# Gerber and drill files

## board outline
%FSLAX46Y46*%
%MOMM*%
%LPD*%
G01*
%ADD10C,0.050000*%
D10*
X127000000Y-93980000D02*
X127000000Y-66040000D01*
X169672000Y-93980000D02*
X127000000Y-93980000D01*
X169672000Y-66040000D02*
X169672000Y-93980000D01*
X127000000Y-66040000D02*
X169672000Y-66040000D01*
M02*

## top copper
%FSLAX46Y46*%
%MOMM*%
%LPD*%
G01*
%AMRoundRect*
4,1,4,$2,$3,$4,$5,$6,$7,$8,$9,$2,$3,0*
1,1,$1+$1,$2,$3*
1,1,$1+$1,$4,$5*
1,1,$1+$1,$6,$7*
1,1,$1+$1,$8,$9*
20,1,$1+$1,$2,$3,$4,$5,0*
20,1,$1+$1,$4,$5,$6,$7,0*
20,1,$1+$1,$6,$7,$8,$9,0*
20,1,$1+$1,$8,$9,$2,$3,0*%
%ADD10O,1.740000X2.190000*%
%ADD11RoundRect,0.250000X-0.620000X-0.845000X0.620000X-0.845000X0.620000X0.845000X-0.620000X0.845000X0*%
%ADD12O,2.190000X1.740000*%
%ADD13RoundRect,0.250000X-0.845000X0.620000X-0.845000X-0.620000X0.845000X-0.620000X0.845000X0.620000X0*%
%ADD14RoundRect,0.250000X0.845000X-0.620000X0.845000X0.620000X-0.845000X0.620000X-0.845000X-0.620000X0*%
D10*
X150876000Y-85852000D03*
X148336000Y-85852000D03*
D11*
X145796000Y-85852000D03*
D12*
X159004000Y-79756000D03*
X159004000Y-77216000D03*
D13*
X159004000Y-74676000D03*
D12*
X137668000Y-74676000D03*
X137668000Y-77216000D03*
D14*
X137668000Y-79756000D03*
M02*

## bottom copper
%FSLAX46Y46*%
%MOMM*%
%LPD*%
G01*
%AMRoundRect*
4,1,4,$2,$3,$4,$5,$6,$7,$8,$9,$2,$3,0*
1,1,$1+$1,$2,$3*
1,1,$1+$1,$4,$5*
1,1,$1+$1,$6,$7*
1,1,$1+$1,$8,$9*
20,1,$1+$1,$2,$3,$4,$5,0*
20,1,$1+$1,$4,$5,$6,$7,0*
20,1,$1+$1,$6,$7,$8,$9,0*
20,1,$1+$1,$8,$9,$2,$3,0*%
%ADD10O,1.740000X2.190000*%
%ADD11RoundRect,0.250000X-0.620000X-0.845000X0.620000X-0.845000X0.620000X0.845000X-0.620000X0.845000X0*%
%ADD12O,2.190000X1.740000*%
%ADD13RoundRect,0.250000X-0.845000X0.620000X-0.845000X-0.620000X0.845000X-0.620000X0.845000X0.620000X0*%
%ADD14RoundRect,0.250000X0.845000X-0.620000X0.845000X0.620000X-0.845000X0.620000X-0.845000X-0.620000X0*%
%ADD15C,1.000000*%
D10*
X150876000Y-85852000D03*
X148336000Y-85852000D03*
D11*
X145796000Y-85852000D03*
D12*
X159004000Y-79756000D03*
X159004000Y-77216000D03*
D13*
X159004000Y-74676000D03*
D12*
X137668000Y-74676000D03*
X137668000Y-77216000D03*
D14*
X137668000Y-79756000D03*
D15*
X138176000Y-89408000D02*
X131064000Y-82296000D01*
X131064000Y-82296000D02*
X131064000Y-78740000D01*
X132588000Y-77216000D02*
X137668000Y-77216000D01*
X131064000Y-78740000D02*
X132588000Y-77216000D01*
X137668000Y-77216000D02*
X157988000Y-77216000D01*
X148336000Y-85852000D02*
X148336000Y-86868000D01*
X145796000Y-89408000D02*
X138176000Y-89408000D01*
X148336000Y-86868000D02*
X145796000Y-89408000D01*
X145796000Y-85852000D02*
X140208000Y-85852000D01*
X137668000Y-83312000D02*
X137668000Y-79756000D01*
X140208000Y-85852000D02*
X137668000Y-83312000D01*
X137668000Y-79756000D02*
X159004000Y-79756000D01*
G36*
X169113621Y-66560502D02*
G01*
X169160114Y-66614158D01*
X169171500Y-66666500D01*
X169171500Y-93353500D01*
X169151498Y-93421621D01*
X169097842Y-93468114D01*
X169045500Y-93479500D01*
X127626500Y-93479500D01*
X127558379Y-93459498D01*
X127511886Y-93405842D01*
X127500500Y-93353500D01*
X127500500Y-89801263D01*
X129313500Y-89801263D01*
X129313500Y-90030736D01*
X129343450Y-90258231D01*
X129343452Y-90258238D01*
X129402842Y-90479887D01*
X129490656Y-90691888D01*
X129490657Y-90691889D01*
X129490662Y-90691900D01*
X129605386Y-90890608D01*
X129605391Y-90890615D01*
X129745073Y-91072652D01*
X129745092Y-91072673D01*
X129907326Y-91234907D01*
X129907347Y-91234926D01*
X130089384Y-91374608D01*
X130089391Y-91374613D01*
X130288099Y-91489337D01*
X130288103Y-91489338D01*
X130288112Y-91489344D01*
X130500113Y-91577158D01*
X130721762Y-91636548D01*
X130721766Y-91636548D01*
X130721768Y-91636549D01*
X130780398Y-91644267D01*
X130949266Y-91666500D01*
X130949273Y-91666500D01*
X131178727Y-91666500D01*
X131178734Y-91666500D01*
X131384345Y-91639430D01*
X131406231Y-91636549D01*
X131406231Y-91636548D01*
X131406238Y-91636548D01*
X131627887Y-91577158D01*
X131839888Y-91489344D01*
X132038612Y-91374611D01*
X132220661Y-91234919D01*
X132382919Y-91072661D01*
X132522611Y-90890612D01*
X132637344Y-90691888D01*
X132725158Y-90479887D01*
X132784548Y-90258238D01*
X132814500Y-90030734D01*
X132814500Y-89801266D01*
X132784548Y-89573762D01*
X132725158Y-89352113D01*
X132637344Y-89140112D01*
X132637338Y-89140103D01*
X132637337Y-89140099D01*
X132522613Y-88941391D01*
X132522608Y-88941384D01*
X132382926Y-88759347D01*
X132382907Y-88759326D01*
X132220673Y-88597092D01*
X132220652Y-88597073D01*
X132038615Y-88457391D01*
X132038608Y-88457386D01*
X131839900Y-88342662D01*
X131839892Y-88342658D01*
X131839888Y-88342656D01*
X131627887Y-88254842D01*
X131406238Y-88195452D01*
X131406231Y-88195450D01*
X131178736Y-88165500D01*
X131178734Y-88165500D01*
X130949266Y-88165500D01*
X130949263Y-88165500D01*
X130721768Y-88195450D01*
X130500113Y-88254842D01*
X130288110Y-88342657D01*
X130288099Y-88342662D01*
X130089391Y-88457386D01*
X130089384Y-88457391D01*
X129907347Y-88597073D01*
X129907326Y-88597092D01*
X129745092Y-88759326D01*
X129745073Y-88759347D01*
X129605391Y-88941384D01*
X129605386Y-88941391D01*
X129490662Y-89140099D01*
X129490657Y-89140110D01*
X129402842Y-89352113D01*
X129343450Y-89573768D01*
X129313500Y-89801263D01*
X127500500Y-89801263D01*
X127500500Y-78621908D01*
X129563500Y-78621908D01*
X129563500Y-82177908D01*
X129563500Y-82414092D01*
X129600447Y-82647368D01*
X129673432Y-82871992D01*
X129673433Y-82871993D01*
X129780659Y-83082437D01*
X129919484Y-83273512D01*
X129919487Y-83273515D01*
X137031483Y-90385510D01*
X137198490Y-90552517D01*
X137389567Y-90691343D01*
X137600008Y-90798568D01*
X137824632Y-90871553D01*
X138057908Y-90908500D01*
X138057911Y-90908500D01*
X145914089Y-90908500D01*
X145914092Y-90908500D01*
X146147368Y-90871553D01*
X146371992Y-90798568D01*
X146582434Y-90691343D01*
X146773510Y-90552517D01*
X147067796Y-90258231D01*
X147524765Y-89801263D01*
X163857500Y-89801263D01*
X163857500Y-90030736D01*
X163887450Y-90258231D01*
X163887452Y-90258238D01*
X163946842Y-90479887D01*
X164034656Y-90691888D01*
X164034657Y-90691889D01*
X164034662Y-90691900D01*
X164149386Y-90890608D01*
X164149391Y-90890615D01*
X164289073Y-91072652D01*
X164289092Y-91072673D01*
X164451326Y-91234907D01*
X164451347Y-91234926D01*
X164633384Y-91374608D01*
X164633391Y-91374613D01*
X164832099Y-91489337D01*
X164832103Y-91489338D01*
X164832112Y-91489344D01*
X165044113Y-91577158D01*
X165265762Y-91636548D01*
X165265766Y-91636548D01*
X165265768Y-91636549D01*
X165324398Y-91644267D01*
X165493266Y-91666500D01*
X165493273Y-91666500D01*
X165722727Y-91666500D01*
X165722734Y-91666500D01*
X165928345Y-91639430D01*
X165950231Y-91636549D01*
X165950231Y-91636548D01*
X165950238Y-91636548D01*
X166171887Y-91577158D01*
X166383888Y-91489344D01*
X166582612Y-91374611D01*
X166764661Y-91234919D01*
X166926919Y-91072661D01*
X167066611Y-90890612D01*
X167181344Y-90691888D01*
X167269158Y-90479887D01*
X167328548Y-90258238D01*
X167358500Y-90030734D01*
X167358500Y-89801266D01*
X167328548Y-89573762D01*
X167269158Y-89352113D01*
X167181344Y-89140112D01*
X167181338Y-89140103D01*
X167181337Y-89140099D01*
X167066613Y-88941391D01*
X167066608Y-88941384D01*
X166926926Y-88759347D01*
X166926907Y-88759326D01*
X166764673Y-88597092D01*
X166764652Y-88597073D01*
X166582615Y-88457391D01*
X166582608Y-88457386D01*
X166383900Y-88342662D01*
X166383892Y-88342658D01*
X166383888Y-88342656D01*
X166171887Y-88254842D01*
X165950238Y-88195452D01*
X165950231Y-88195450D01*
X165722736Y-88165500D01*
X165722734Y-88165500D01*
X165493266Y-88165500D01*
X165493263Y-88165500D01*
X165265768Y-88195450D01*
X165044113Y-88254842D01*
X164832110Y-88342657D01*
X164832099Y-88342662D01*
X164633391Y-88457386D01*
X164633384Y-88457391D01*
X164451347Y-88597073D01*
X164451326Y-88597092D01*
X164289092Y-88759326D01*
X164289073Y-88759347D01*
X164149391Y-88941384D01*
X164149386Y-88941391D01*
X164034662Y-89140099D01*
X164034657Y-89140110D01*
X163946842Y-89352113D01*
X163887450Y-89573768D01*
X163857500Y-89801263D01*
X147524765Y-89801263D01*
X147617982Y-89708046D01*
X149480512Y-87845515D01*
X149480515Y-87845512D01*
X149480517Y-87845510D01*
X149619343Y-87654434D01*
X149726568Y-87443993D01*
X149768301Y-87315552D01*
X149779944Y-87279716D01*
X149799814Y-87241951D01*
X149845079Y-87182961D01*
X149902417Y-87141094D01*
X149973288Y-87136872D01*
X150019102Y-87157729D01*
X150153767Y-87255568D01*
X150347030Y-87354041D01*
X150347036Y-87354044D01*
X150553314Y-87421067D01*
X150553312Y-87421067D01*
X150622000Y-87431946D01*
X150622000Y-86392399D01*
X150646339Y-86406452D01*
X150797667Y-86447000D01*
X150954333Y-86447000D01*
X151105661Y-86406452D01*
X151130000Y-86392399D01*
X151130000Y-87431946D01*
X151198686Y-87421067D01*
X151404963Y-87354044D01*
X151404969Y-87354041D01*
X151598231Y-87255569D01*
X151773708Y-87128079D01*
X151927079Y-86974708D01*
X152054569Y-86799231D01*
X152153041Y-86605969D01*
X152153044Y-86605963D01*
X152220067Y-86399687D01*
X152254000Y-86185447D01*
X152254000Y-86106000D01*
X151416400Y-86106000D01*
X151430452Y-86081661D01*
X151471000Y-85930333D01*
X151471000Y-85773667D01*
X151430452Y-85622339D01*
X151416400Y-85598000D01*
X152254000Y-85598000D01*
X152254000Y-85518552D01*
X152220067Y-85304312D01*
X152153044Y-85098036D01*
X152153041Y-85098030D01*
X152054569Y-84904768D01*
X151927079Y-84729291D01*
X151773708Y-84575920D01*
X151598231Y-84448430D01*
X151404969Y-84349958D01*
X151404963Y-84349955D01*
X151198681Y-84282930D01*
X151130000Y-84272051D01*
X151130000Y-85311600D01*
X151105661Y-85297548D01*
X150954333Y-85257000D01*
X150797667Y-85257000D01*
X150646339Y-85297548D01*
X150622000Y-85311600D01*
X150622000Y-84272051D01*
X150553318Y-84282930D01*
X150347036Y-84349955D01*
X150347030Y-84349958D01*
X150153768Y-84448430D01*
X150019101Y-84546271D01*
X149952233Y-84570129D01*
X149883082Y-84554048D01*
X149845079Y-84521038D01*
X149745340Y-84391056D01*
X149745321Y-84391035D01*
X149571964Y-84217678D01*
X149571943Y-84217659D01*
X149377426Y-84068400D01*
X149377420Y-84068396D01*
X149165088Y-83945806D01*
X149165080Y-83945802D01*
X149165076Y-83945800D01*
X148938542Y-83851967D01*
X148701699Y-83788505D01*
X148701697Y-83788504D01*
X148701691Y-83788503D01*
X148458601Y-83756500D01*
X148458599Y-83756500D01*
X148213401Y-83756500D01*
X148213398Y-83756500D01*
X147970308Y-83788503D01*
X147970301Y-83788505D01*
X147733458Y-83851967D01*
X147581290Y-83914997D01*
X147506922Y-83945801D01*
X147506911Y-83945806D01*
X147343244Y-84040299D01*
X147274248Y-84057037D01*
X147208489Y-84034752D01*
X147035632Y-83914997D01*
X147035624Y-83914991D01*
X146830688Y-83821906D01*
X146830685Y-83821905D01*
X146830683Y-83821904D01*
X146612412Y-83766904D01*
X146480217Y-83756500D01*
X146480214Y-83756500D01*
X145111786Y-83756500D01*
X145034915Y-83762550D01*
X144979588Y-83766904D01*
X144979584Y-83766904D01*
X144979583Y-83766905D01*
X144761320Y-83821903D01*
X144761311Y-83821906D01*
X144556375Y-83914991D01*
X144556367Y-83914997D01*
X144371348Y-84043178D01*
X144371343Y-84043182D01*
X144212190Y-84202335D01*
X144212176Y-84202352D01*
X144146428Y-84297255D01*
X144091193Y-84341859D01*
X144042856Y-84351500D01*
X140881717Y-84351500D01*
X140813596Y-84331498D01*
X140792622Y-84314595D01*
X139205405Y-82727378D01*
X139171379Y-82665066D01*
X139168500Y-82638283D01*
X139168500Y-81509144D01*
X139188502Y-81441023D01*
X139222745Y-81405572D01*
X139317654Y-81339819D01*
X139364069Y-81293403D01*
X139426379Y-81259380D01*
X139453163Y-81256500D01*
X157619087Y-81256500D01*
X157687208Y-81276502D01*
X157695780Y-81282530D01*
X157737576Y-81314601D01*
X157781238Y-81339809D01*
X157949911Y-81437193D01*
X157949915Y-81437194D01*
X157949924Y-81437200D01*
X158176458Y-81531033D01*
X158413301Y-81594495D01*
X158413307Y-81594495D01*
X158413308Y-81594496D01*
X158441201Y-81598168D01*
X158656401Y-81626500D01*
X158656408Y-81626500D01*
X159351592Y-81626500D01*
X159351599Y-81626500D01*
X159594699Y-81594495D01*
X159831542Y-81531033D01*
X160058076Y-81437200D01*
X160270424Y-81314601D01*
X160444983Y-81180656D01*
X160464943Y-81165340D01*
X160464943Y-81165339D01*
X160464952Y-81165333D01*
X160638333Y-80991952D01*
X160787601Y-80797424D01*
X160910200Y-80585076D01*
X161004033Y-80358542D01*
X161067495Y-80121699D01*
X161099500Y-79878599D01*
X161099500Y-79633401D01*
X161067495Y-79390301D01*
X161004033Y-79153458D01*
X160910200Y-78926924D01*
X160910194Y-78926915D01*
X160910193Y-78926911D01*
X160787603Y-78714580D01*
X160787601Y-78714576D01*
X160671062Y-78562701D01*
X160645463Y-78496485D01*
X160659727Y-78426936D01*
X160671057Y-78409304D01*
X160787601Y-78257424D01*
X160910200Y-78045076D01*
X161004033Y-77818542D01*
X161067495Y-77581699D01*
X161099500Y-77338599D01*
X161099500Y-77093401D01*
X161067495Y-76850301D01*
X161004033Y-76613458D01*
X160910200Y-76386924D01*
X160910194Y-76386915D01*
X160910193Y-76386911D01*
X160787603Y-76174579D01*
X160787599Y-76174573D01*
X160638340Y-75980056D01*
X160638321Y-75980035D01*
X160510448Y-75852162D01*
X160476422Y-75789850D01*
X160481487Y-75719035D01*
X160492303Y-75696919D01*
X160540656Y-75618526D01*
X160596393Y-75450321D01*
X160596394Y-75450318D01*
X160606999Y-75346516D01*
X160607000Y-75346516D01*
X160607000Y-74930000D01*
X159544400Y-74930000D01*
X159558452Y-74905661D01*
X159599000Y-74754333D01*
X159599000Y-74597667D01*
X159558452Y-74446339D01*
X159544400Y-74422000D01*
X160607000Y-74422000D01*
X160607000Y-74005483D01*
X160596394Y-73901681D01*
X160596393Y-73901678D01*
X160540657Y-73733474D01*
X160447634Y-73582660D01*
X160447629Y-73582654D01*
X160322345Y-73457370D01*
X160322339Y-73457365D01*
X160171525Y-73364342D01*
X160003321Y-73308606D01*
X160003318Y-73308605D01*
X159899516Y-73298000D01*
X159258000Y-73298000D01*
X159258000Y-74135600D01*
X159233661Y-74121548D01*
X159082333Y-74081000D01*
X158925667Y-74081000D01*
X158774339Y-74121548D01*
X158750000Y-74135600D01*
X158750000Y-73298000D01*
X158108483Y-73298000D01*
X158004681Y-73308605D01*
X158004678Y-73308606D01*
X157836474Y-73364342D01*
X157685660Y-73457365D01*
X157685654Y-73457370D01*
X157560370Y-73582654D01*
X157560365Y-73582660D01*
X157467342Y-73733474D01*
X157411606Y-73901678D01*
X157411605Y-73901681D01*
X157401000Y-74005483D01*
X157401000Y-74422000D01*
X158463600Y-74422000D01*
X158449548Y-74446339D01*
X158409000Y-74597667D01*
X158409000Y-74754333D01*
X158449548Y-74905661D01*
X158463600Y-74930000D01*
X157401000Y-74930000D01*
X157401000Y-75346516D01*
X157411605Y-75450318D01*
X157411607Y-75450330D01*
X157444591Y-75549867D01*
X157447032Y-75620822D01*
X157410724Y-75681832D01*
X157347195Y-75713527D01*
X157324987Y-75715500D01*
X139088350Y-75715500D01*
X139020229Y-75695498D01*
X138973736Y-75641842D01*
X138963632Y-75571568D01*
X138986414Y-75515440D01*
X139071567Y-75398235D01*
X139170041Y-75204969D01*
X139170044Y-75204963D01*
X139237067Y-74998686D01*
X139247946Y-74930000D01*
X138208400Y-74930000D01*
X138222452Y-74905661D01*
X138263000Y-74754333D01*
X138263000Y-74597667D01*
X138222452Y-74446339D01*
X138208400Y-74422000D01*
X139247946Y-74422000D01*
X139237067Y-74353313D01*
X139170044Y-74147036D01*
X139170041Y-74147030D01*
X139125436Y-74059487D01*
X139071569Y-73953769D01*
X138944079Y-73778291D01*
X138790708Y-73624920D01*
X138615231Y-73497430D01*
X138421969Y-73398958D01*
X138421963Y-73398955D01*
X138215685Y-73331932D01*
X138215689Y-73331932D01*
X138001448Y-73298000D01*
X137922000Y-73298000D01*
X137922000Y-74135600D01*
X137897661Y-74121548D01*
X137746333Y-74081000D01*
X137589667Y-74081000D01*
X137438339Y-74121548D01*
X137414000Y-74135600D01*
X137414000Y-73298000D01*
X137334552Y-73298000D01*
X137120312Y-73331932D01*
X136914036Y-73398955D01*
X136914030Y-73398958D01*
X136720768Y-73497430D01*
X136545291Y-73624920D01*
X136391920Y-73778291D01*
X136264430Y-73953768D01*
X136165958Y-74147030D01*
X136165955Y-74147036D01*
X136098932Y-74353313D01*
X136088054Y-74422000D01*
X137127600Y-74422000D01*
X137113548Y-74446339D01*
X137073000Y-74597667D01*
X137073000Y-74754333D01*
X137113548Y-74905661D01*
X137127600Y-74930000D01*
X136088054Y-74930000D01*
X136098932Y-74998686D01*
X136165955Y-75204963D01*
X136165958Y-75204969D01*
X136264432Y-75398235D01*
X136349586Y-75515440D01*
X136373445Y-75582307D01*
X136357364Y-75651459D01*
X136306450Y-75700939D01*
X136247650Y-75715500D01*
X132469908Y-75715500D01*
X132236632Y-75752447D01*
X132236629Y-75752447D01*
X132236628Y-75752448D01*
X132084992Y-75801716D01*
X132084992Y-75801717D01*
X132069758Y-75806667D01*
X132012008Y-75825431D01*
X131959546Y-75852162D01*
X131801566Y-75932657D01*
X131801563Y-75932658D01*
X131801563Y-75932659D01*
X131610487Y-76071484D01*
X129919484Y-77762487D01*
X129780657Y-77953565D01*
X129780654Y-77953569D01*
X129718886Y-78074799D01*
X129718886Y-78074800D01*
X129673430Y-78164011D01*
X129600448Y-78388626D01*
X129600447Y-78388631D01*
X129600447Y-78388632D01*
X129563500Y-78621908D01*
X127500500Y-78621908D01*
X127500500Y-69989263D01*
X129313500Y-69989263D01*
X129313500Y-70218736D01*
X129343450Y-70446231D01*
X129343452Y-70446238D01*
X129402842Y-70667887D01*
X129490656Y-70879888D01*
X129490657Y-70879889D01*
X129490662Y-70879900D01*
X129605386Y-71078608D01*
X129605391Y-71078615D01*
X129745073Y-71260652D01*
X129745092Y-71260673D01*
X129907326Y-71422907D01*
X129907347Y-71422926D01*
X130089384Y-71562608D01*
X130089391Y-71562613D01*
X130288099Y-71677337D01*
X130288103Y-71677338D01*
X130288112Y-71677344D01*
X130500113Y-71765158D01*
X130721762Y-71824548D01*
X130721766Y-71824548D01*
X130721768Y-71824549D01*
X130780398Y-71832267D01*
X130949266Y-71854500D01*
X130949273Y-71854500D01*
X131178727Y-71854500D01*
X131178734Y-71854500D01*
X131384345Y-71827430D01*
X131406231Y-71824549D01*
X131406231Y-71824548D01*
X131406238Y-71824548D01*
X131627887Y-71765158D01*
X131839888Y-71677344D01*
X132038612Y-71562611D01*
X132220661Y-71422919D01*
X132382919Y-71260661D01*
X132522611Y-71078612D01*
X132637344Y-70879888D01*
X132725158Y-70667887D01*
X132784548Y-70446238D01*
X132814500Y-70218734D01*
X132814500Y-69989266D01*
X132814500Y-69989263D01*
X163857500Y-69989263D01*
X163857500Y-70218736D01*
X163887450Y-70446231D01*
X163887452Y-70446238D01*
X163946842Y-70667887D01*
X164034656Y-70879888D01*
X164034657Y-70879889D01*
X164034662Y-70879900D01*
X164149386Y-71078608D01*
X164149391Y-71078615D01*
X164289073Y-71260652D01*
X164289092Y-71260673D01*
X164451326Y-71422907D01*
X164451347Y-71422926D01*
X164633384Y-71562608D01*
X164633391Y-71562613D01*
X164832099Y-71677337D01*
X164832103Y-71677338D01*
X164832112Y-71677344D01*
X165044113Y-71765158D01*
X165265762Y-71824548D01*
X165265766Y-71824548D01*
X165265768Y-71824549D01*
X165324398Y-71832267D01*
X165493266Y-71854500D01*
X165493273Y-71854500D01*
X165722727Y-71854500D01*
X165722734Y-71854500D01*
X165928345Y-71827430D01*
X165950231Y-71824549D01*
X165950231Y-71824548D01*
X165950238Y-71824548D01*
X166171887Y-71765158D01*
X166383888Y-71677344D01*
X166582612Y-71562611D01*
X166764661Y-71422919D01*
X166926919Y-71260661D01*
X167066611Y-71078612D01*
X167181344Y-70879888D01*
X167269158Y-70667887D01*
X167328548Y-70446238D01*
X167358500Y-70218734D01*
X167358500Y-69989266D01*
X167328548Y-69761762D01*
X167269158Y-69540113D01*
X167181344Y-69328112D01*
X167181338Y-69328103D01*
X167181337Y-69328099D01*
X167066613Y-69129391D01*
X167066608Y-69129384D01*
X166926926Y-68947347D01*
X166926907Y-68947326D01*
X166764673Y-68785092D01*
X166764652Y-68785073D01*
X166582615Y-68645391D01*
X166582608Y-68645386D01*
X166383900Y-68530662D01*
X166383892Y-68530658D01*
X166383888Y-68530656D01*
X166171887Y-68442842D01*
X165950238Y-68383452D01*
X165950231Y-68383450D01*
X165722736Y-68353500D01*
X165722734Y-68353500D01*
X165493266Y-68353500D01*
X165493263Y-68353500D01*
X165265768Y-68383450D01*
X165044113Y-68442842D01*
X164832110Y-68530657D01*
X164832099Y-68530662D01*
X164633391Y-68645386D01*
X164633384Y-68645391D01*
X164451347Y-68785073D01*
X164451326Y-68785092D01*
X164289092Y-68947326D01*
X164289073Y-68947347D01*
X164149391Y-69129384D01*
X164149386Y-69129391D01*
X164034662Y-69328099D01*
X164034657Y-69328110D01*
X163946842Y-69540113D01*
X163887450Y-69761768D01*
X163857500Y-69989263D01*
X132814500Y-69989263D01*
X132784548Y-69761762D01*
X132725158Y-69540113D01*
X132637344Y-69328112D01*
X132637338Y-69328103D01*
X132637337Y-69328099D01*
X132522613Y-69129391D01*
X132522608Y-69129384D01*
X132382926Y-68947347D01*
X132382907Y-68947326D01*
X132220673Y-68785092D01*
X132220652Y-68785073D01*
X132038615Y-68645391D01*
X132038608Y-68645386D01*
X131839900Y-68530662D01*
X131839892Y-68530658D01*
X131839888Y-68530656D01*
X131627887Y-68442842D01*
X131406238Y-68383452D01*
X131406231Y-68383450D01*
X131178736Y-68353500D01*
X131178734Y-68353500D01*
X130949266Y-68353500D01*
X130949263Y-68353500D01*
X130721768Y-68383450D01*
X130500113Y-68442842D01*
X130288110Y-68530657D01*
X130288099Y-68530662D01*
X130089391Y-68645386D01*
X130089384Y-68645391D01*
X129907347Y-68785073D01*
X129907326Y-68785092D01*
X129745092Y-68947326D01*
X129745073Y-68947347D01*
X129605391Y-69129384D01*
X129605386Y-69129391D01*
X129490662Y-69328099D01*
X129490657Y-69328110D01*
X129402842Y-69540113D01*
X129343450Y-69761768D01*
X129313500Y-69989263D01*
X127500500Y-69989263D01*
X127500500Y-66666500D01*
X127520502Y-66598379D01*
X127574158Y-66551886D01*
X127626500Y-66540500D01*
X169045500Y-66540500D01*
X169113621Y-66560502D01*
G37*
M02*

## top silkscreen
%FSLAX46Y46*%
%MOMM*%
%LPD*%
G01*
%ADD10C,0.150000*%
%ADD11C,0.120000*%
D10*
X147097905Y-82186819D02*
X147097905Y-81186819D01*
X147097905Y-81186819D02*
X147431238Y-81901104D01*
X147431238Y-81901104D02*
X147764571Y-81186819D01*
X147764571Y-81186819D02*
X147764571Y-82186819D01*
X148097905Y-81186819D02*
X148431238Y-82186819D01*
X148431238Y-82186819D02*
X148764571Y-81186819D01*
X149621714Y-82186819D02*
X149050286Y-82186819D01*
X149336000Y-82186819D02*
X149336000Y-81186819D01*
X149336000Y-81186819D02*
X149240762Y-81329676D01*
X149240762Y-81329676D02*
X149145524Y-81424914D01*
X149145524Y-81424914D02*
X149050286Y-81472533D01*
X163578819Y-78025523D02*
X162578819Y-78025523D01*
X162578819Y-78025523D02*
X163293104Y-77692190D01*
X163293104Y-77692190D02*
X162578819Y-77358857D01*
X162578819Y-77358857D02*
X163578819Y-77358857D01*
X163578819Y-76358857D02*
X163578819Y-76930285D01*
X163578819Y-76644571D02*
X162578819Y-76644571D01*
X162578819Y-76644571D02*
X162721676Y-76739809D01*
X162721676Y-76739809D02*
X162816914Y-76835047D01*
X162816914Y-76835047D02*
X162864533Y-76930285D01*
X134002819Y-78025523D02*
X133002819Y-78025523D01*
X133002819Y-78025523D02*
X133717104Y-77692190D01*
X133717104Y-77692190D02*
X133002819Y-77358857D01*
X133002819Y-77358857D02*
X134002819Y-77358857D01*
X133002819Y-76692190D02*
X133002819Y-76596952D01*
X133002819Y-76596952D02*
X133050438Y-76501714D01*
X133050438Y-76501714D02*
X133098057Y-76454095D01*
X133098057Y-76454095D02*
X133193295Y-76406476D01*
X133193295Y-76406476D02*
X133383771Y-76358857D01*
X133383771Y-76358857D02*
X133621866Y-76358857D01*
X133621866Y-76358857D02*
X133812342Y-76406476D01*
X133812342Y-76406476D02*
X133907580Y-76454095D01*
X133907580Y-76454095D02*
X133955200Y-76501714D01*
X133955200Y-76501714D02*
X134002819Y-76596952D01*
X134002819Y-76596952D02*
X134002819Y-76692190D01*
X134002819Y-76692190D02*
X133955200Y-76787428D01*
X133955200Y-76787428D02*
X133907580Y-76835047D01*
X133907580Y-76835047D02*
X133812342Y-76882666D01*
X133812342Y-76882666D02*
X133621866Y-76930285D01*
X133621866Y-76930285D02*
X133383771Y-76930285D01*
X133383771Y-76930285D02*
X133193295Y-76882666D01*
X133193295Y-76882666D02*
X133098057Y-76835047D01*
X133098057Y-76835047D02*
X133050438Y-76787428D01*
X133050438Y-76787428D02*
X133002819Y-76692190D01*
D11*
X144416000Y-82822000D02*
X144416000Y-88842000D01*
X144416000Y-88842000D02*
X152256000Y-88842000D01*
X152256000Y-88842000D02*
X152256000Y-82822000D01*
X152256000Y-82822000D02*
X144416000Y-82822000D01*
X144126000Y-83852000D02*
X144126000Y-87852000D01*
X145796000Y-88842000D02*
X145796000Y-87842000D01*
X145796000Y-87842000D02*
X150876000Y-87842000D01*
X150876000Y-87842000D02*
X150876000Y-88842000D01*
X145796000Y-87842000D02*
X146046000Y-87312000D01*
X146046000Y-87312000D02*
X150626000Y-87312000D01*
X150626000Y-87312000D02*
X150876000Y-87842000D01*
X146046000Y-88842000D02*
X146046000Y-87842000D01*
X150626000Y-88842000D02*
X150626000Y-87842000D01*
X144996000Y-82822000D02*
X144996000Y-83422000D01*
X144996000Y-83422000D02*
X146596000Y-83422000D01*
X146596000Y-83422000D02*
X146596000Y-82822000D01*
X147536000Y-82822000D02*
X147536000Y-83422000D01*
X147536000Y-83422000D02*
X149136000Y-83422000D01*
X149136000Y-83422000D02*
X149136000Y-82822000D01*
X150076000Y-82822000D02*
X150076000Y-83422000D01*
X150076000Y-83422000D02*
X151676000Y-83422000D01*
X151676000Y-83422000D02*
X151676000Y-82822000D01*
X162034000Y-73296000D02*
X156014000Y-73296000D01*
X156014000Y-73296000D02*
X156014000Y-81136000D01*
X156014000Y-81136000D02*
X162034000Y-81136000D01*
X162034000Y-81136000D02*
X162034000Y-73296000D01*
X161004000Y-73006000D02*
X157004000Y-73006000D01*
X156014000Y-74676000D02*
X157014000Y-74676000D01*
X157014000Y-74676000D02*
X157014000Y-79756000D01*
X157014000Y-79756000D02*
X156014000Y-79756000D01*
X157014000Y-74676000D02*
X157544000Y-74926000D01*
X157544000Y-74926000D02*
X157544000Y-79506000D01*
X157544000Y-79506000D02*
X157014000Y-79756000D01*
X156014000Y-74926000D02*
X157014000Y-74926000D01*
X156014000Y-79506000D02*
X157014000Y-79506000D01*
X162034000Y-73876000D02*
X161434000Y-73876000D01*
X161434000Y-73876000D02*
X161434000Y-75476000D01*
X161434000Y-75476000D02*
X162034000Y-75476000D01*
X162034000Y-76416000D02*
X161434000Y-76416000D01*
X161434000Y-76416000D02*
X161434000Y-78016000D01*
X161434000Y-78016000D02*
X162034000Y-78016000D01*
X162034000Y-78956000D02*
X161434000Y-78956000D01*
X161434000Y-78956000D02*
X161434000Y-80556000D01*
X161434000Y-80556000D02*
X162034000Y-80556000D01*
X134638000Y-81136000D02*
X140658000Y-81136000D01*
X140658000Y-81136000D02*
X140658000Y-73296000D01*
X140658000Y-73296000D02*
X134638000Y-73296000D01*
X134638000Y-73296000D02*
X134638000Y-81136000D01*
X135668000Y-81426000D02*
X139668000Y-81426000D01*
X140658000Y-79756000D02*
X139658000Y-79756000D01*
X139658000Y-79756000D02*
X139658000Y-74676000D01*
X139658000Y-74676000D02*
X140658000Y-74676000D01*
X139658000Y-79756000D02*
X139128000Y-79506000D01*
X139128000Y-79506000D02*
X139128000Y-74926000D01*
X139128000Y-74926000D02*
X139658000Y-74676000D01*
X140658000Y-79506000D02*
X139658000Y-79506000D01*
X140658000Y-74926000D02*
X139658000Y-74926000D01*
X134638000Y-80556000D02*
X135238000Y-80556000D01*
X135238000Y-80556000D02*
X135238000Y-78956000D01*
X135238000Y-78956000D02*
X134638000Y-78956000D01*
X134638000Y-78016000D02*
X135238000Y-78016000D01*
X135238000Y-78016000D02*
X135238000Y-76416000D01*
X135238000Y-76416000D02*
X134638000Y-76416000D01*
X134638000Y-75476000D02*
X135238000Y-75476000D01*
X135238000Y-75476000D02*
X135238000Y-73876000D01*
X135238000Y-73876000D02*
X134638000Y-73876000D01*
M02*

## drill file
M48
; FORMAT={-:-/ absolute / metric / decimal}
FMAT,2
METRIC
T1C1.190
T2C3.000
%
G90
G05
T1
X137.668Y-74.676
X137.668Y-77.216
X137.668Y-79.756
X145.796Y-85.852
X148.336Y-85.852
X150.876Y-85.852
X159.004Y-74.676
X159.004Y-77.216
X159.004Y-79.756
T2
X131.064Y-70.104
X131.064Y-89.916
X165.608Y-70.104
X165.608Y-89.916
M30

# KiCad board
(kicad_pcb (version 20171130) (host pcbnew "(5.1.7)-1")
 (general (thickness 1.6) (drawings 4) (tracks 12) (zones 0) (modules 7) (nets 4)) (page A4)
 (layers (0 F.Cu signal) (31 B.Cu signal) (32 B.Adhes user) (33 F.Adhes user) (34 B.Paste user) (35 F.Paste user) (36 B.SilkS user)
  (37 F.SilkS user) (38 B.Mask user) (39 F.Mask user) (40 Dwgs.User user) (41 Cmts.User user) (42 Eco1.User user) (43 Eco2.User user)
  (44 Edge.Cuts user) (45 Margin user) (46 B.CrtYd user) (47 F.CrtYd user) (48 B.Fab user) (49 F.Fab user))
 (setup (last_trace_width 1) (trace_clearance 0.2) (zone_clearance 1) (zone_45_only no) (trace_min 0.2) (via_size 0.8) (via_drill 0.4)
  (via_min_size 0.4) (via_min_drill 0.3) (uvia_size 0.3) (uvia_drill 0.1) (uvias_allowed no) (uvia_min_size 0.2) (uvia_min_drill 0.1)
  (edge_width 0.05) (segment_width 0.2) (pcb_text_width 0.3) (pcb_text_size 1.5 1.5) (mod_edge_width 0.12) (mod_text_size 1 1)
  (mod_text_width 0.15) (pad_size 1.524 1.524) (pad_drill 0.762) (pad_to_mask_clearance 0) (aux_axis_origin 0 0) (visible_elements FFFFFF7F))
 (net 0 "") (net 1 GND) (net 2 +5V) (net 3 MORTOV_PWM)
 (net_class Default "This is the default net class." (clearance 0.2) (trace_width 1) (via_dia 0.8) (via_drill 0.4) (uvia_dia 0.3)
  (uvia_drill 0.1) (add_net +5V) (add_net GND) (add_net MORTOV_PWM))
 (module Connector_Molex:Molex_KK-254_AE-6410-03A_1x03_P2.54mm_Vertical (layer F.Cu) (at 145.796 85.852)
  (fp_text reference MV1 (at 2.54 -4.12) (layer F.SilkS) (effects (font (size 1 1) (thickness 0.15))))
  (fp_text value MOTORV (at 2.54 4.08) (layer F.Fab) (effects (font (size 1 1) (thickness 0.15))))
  (fp_line (start -1.38 -3.03) (end -1.38 2.99) (layer F.SilkS) (width 0.12))
  (fp_line (start -1.38 2.99) (end 6.46 2.99) (layer F.SilkS) (width 0.12))
  (fp_line (start 6.46 2.99) (end 6.46 -3.03) (layer F.SilkS) (width 0.12))
  (fp_line (start 6.46 -3.03) (end -1.38 -3.03) (layer F.SilkS) (width 0.12))
  (fp_line (start -1.67 -2) (end -1.67 2) (layer F.SilkS) (width 0.12))
  (fp_line (start 0 2.99) (end 0 1.99) (layer F.SilkS) (width 0.12))
  (fp_line (start 0 1.99) (end 5.08 1.99) (layer F.SilkS) (width 0.12))
  (fp_line (start 5.08 1.99) (end 5.08 2.99) (layer F.SilkS) (width 0.12))
  (fp_line (start 0 1.99) (end 0.25 1.46) (layer F.SilkS) (width 0.12))
  (fp_line (start 0.25 1.46) (end 4.83 1.46) (layer F.SilkS) (width 0.12))
  (fp_line (start 4.83 1.46) (end 5.08 1.99) (layer F.SilkS) (width 0.12))
  (fp_line (start 0.25 2.99) (end 0.25 1.99) (layer F.SilkS) (width 0.12))
  (fp_line (start 4.83 2.99) (end 4.83 1.99) (layer F.SilkS) (width 0.12))
  (fp_line (start -0.8 -3.03) (end -0.8 -2.43) (layer F.SilkS) (width 0.12))
  (fp_line (start -0.8 -2.43) (end 0.8 -2.43) (layer F.SilkS) (width 0.12))
  (fp_line (start 0.8 -2.43) (end 0.8 -3.03) (layer F.SilkS) (width 0.12))
  (fp_line (start 1.74 -3.03) (end 1.74 -2.43) (layer F.SilkS) (width 0.12))
  (fp_line (start 1.74 -2.43) (end 3.34 -2.43) (layer F.SilkS) (width 0.12))
  (fp_line (start 3.34 -2.43) (end 3.34 -3.03) (layer F.SilkS) (width 0.12))
  (fp_line (start 4.28 -3.03) (end 4.28 -2.43) (layer F.SilkS) (width 0.12))
  (fp_line (start 4.28 -2.43) (end 5.88 -2.43) (layer F.SilkS) (width 0.12))
  (fp_line (start 5.88 -2.43) (end 5.88 -3.03) (layer F.SilkS) (width 0.12))
  (pad 3 thru_hole oval (at 5.08 0) (size 1.74 2.19) (drill 1.19) (layers *.Cu *.Mask) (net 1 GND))
  (pad 2 thru_hole oval (at 2.54 0) (size 1.74 2.19) (drill 1.19) (layers *.Cu *.Mask) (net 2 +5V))
  (pad 1 thru_hole roundrect (at 0 0) (size 1.74 2.19) (drill 1.19) (layers *.Cu *.Mask) (roundrect_rratio 0.143678) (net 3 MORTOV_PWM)))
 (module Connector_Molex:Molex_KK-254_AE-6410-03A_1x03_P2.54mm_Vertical (layer F.Cu) (at 159.004 74.676 270)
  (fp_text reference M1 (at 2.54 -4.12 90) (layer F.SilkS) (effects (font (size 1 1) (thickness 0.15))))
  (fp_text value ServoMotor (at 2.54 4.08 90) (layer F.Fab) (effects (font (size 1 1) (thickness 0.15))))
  (fp_line (start -1.38 -3.03) (end -1.38 2.99) (layer F.SilkS) (width 0.12))
  (fp_line (start -1.38 2.99) (end 6.46 2.99) (layer F.SilkS) (width 0.12))
  (fp_line (start 6.46 2.99) (end 6.46 -3.03) (layer F.SilkS) (width 0.12))
  (fp_line (start 6.46 -3.03) (end -1.38 -3.03) (layer F.SilkS) (width 0.12))
  (fp_line (start -1.67 -2) (end -1.67 2) (layer F.SilkS) (width 0.12))
  (fp_line (start 0 2.99) (end 0 1.99) (layer F.SilkS) (width 0.12))
  (fp_line (start 0 1.99) (end 5.08 1.99) (layer F.SilkS) (width 0.12))
  (fp_line (start 5.08 1.99) (end 5.08 2.99) (layer F.SilkS) (width 0.12))
  (fp_line (start 0 1.99) (end 0.25 1.46) (layer F.SilkS) (width 0.12))
  (fp_line (start 0.25 1.46) (end 4.83 1.46) (layer F.SilkS) (width 0.12))
  (fp_line (start 4.83 1.46) (end 5.08 1.99) (layer F.SilkS) (width 0.12))
  (fp_line (start 0.25 2.99) (end 0.25 1.99) (layer F.SilkS) (width 0.12))
  (fp_line (start 4.83 2.99) (end 4.83 1.99) (layer F.SilkS) (width 0.12))
  (fp_line (start -0.8 -3.03) (end -0.8 -2.43) (layer F.SilkS) (width 0.12))
  (fp_line (start -0.8 -2.43) (end 0.8 -2.43) (layer F.SilkS) (width 0.12))
  (fp_line (start 0.8 -2.43) (end 0.8 -3.03) (layer F.SilkS) (width 0.12))
  (fp_line (start 1.74 -3.03) (end 1.74 -2.43) (layer F.SilkS) (width 0.12))
  (fp_line (start 1.74 -2.43) (end 3.34 -2.43) (layer F.SilkS) (width 0.12))
  (fp_line (start 3.34 -2.43) (end 3.34 -3.03) (layer F.SilkS) (width 0.12))
  (fp_line (start 4.28 -3.03) (end 4.28 -2.43) (layer F.SilkS) (width 0.12))
  (fp_line (start 4.28 -2.43) (end 5.88 -2.43) (layer F.SilkS) (width 0.12))
  (fp_line (start 5.88 -2.43) (end 5.88 -3.03) (layer F.SilkS) (width 0.12))
  (pad 3 thru_hole oval (at 5.08 0 270) (size 1.74 2.19) (drill 1.19) (layers *.Cu *.Mask) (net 3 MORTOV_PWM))
  (pad 2 thru_hole oval (at 2.54 0 270) (size 1.74 2.19) (drill 1.19) (layers *.Cu *.Mask) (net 2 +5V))
  (pad 1 thru_hole roundrect (at 0 0 270) (size 1.74 2.19) (drill 1.19) (layers *.Cu *.Mask) (roundrect_rratio 0.143678) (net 1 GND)))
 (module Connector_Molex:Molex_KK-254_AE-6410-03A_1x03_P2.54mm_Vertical (layer F.Cu) (at 137.668 79.756 90)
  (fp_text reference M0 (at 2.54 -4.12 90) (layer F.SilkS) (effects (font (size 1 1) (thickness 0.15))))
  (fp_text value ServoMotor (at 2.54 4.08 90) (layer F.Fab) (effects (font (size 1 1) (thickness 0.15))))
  (fp_line (start -1.38 -3.03) (end -1.38 2.99) (layer F.SilkS) (width 0.12))
  (fp_line (start -1.38 2.99) (end 6.46 2.99) (layer F.SilkS) (width 0.12))
  (fp_line (start 6.46 2.99) (end 6.46 -3.03) (layer F.SilkS) (width 0.12))
  (fp_line (start 6.46 -3.03) (end -1.38 -3.03) (layer F.SilkS) (width 0.12))
  (fp_line (start -1.67 -2) (end -1.67 2) (layer F.SilkS) (width 0.12))
  (fp_line (start 0 2.99) (end 0 1.99) (layer F.SilkS) (width 0.12))
  (fp_line (start 0 1.99) (end 5.08 1.99) (layer F.SilkS) (width 0.12))
  (fp_line (start 5.08 1.99) (end 5.08 2.99) (layer F.SilkS) (width 0.12))
  (fp_line (start 0 1.99) (end 0.25 1.46) (layer F.SilkS) (width 0.12))
  (fp_line (start 0.25 1.46) (end 4.83 1.46) (layer F.SilkS) (width 0.12))
  (fp_line (start 4.83 1.46) (end 5.08 1.99) (layer F.SilkS) (width 0.12))
  (fp_line (start 0.25 2.99) (end 0.25 1.99) (layer F.SilkS) (width 0.12))
  (fp_line (start 4.83 2.99) (end 4.83 1.99) (layer F.SilkS) (width 0.12))
  (fp_line (start -0.8 -3.03) (end -0.8 -2.43) (layer F.SilkS) (width 0.12))
  (fp_line (start -0.8 -2.43) (end 0.8 -2.43) (layer F.SilkS) (width 0.12))
  (fp_line (start 0.8 -2.43) (end 0.8 -3.03) (layer F.SilkS) (width 0.12))
  (fp_line (start 1.74 -3.03) (end 1.74 -2.43) (layer F.SilkS) (width 0.12))
  (fp_line (start 1.74 -2.43) (end 3.34 -2.43) (layer F.SilkS) (width 0.12))
  (fp_line (start 3.34 -2.43) (end 3.34 -3.03) (layer F.SilkS) (width 0.12))
  (fp_line (start 4.28 -3.03) (end 4.28 -2.43) (layer F.SilkS) (width 0.12))
  (fp_line (start 4.28 -2.43) (end 5.88 -2.43) (layer F.SilkS) (width 0.12))
  (fp_line (start 5.88 -2.43) (end 5.88 -3.03) (layer F.SilkS) (width 0.12))
  (pad 3 thru_hole oval (at 5.08 0 90) (size 1.74 2.19) (drill 1.19) (layers *.Cu *.Mask) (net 1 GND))
  (pad 2 thru_hole oval (at 2.54 0 90) (size 1.74 2.19) (drill 1.19) (layers *.Cu *.Mask) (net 2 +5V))
  (pad 1 thru_hole roundrect (at 0 0 90) (size 1.74 2.19) (drill 1.19) (layers *.Cu *.Mask) (roundrect_rratio 0.143678) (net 3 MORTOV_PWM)))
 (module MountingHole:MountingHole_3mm (layer F.Cu) (at 131.064 70.104)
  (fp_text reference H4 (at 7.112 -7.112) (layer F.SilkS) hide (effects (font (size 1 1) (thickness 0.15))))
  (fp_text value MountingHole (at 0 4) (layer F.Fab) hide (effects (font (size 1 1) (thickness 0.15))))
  (pad 1 np_thru_hole circle (at 0 0) (size 3 3) (drill 3) (layers *.Cu *.Mask)))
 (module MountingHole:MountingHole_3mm (layer F.Cu) (at 165.608 89.916)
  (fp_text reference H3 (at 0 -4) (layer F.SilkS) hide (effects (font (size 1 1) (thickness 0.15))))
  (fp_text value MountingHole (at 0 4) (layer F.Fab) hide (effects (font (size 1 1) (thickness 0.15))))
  (pad 1 np_thru_hole circle (at 0 0) (size 3 3) (drill 3) (layers *.Cu *.Mask)))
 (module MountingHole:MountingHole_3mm (layer F.Cu) (at 165.608 70.104)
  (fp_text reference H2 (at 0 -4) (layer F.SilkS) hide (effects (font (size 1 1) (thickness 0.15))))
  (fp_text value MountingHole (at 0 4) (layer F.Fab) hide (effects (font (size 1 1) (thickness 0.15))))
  (pad 1 np_thru_hole circle (at 0 0) (size 3 3) (drill 3) (layers *.Cu *.Mask)))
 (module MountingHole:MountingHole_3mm (layer F.Cu) (at 131.064 89.916)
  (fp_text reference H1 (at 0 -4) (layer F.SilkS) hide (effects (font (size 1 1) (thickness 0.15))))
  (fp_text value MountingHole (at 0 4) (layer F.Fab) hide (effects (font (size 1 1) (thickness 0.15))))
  (pad 1 np_thru_hole circle (at 0 0) (size 3 3) (drill 3) (layers *.Cu *.Mask)))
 (gr_line (start 127 93.98) (end 127 66.04) (layer Edge.Cuts) (width 0.05))
 (gr_line (start 169.672 93.98) (end 127 93.98) (layer Edge.Cuts) (width 0.05))
 (gr_line (start 169.672 66.04) (end 169.672 93.98) (layer Edge.Cuts) (width 0.05))
 (gr_line (start 127 66.04) (end 169.672 66.04) (layer Edge.Cuts) (width 0.05))
 (segment (start 138.176 89.408) (end 131.064 82.296) (width 1) (layer B.Cu) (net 2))
 (segment (start 131.064 82.296) (end 131.064 78.74) (width 1) (layer B.Cu) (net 2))
 (segment (start 132.588 77.216) (end 137.668 77.216) (width 1) (layer B.Cu) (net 2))
 (segment (start 131.064 78.74) (end 132.588 77.216) (width 1) (layer B.Cu) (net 2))
 (segment (start 137.668 77.216) (end 157.988 77.216) (width 1) (layer B.Cu) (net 2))
 (segment (start 148.336 85.852) (end 148.336 86.868) (width 1) (layer B.Cu) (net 2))
 (segment (start 145.796 89.408) (end 138.176 89.408) (width 1) (layer B.Cu) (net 2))
 (segment (start 148.336 86.868) (end 145.796 89.408) (width 1) (layer B.Cu) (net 2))
 (segment (start 145.796 85.852) (end 140.208 85.852) (width 1) (layer B.Cu) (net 3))
 (segment (start 137.668 83.312) (end 137.668 79.756) (width 1) (layer B.Cu) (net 3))
 (segment (start 140.208 85.852) (end 137.668 83.312) (width 1) (layer B.Cu) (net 3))
 (segment (start 137.668 79.756) (end 159.004 79.756) (width 1) (layer B.Cu) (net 3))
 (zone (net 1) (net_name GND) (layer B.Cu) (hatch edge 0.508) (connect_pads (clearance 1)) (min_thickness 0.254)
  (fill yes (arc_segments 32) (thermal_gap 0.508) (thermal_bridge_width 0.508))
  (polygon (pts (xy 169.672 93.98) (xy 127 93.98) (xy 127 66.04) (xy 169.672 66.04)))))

